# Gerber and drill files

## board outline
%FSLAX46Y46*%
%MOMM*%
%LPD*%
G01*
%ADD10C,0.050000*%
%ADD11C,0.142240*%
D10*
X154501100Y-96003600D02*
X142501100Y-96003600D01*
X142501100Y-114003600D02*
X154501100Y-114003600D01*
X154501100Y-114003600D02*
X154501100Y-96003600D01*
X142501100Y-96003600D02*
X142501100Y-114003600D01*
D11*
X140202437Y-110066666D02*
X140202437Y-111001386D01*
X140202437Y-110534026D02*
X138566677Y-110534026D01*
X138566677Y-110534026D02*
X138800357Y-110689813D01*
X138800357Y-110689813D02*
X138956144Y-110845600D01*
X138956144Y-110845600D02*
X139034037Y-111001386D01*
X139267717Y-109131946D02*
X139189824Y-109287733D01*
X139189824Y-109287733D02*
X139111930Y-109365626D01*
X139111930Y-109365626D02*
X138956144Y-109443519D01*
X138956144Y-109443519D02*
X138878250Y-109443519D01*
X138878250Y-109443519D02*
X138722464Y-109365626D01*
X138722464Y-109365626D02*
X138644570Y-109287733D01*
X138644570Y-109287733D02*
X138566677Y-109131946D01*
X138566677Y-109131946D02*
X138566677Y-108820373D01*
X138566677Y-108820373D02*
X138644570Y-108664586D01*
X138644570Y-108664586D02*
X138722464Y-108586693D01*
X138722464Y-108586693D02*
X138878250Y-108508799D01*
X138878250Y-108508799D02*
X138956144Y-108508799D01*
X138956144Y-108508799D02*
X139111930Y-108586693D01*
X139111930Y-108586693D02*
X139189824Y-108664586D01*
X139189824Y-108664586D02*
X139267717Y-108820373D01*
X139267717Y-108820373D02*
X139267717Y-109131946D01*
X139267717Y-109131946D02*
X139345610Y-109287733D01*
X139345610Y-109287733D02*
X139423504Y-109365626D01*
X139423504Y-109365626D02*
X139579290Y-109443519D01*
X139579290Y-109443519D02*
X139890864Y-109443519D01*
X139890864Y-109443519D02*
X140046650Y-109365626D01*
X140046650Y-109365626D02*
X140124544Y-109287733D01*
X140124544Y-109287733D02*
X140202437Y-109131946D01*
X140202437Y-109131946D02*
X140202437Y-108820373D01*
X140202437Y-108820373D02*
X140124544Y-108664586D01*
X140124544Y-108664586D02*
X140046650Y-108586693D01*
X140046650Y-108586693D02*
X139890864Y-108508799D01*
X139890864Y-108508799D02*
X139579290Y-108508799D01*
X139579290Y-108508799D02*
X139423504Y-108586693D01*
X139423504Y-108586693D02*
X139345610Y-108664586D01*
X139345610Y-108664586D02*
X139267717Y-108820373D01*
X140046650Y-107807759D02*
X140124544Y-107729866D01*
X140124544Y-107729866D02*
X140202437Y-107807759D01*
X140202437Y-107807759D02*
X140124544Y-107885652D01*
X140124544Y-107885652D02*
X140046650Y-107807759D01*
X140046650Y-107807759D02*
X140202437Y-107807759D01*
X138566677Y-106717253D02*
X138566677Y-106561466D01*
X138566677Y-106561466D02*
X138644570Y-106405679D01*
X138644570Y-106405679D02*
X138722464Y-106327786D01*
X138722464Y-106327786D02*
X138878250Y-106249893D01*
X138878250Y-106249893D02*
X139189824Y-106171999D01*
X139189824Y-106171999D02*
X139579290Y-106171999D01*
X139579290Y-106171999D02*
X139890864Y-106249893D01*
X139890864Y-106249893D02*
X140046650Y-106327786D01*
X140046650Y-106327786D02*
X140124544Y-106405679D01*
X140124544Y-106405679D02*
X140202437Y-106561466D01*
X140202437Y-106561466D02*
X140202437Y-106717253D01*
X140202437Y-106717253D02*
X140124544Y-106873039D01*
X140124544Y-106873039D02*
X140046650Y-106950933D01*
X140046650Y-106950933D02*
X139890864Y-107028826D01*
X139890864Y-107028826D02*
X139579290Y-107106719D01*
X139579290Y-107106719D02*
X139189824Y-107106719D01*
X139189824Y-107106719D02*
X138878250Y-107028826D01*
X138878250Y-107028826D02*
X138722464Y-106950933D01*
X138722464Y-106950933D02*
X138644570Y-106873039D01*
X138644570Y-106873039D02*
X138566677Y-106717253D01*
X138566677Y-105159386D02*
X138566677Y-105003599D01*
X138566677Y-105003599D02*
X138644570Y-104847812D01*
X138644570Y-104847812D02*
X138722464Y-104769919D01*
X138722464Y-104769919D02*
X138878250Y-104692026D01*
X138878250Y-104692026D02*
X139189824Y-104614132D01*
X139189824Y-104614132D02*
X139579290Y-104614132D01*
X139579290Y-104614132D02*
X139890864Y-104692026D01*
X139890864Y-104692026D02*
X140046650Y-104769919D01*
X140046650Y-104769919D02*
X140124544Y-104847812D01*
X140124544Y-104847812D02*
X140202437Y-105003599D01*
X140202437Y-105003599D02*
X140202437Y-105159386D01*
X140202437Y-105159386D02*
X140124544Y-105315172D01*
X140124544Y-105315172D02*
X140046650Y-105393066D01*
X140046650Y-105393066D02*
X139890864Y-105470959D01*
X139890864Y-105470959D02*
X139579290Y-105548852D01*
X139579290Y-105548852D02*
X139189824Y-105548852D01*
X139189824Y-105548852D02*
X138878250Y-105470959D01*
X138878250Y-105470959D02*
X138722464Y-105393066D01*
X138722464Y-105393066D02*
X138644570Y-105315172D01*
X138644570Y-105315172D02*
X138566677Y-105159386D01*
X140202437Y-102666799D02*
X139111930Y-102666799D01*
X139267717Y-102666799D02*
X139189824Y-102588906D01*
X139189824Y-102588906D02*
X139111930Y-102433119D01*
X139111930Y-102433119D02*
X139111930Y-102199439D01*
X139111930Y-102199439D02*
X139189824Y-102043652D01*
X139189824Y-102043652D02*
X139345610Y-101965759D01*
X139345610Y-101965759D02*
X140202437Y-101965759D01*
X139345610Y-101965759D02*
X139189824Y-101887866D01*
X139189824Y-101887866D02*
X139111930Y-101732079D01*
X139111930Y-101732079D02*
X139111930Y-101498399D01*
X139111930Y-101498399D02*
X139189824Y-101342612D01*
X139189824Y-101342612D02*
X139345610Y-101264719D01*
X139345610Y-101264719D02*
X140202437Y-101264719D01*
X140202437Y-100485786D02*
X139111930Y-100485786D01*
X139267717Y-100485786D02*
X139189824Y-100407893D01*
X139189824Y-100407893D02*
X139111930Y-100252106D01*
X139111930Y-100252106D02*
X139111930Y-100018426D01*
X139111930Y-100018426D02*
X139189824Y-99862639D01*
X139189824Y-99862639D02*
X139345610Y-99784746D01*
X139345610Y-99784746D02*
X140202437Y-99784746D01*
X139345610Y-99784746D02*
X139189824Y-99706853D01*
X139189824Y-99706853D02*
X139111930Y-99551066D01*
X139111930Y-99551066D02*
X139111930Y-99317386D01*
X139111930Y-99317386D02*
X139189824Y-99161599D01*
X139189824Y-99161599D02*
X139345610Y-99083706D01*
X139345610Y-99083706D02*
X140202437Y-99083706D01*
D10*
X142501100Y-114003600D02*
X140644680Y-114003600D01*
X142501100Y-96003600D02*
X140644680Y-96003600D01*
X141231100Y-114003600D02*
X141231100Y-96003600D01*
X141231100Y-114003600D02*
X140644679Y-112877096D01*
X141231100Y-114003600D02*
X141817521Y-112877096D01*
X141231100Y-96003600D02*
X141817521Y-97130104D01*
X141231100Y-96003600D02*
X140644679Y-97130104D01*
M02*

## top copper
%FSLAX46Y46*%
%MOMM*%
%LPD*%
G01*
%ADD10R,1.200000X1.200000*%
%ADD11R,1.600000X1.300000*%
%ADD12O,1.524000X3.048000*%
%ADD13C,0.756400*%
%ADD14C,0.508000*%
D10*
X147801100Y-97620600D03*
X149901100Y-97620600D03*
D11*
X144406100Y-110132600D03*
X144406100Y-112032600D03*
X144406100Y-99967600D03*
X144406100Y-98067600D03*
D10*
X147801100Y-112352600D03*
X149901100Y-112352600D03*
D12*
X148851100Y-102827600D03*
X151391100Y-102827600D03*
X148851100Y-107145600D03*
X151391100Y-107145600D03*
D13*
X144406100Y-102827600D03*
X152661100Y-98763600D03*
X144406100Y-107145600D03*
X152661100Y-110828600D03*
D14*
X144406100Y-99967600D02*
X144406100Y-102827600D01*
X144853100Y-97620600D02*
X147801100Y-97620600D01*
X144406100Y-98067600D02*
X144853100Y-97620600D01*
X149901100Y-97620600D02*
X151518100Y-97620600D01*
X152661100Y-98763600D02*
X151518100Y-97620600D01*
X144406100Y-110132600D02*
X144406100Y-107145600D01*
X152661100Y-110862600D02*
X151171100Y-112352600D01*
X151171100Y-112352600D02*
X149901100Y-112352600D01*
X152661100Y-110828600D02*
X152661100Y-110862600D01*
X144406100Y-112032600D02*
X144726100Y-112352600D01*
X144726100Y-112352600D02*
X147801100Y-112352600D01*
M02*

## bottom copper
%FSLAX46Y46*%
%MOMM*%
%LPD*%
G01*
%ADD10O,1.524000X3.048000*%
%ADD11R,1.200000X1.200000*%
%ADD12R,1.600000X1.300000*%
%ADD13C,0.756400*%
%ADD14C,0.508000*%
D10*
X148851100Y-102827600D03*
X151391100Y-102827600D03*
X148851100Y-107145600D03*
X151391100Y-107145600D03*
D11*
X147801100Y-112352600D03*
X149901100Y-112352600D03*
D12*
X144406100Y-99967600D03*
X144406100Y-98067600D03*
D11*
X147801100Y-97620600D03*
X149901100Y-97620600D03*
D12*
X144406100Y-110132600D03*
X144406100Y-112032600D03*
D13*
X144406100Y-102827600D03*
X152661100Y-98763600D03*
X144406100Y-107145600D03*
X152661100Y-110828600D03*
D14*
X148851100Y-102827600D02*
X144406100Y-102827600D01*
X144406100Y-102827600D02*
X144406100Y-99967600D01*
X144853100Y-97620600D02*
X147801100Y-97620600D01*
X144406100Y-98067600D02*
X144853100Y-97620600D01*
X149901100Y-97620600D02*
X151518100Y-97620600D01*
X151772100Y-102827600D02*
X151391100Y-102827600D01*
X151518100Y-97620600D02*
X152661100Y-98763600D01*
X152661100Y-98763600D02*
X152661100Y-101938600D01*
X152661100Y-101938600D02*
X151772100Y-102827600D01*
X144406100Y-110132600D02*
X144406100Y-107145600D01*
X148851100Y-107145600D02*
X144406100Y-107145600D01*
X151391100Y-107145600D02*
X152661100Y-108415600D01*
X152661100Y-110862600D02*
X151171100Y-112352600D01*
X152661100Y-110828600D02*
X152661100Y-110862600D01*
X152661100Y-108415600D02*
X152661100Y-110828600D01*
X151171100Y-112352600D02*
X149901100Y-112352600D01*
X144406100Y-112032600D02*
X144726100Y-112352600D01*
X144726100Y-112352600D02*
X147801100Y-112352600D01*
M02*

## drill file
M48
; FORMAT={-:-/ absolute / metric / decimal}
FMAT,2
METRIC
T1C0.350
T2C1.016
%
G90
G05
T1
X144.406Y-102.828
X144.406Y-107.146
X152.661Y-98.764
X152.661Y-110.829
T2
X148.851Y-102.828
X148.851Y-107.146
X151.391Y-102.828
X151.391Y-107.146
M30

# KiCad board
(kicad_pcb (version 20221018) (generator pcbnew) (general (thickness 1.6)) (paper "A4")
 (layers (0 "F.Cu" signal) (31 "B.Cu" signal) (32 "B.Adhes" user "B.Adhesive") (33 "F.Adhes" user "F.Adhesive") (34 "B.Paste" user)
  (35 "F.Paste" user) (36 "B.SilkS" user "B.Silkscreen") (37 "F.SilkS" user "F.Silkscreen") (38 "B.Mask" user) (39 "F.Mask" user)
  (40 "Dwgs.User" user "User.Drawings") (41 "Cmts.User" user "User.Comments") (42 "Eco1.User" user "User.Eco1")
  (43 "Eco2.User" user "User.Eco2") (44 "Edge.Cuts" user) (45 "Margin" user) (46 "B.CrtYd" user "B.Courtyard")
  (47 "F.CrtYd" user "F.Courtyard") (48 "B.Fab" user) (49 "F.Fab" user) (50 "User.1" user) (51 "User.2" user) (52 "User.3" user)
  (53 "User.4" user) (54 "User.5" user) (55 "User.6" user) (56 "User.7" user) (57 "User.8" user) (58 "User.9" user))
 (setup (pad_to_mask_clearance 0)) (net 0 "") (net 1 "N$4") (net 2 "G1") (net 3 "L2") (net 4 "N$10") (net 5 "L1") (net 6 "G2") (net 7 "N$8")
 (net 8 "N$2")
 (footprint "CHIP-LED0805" (layer "F.Cu") (at 148.8511 97.6206 -90)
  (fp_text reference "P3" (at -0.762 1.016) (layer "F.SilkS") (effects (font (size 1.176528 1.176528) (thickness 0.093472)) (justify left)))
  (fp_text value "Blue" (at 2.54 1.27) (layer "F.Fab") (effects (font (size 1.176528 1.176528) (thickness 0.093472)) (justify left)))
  (pad "A" smd rect (at 0 1.05 270) (size 1.2 1.2) (layers "F.Cu" "F.Paste" "F.Mask") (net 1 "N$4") (solder_mask_margin 0.1016)
   (thermal_bridge_angle 45))
  (pad "C" smd rect (at 0 -1.05 270) (size 1.2 1.2) (layers "F.Cu" "F.Paste" "F.Mask") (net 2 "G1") (solder_mask_margin 0.1016)
   (thermal_bridge_angle 45)))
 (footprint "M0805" (layer "F.Cu") (at 144.4061 111.0826 -90)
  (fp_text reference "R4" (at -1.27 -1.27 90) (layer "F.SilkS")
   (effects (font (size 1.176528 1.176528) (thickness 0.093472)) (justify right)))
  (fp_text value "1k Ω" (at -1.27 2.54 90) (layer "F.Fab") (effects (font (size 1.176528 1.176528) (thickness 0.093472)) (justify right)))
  (pad "1" smd rect (at -0.95 0 270) (size 1.3 1.6) (layers "F.Cu" "F.Paste" "F.Mask") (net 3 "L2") (solder_mask_margin 0.1016)
   (thermal_bridge_angle 45))
  (pad "2" smd rect (at 0.95 0 270) (size 1.3 1.6) (layers "F.Cu" "F.Paste" "F.Mask") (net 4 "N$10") (solder_mask_margin 0.1016)
   (thermal_bridge_angle 45)))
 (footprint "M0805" (layer "F.Cu") (at 144.4061 99.0176 90)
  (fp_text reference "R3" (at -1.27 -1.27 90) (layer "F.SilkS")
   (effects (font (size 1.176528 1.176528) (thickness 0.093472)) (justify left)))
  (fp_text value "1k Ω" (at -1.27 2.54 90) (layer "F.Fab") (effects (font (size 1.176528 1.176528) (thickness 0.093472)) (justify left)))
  (pad "1" smd rect (at -0.95 0 90) (size 1.3 1.6) (layers "F.Cu" "F.Paste" "F.Mask") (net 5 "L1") (solder_mask_margin 0.1016)
   (thermal_bridge_angle 45))
  (pad "2" smd rect (at 0.95 0 90) (size 1.3 1.6) (layers "F.Cu" "F.Paste" "F.Mask") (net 1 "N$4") (solder_mask_margin 0.1016)
   (thermal_bridge_angle 45)))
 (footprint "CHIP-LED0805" (layer "F.Cu") (at 148.8511 112.3526 -90)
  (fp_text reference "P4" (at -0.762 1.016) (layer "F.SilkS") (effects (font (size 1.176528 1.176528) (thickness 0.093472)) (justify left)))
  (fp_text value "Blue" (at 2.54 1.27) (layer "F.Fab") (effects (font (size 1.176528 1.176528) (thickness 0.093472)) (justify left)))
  (pad "A" smd rect (at 0 1.05 270) (size 1.2 1.2) (layers "F.Cu" "F.Paste" "F.Mask") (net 4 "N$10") (solder_mask_margin 0.1016)
   (thermal_bridge_angle 45))
  (pad "C" smd rect (at 0 -1.05 270) (size 1.2 1.2) (layers "F.Cu" "F.Paste" "F.Mask") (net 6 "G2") (solder_mask_margin 0.1016)
   (thermal_bridge_angle 45)))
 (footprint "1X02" (layer "F.Cu") (at 150.1211 102.8276)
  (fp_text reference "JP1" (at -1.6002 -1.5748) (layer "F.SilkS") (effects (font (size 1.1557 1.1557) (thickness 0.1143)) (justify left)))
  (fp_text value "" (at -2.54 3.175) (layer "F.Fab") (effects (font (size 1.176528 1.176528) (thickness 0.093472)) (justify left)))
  (pad "1" thru_hole oval (at -1.27 0 90) (size 3.048 1.524) (drill 1.016) (layers "*.Cu" "*.Mask") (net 5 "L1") (solder_mask_margin 0.1016)
   (thermal_bridge_angle 45))
  (pad "2" thru_hole oval (at 1.27 0 90) (size 3.048 1.524) (drill 1.016) (layers "*.Cu" "*.Mask") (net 2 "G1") (solder_mask_margin 0.1016)
   (thermal_bridge_angle 45)))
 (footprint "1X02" (layer "F.Cu") (at 150.1211 107.1456)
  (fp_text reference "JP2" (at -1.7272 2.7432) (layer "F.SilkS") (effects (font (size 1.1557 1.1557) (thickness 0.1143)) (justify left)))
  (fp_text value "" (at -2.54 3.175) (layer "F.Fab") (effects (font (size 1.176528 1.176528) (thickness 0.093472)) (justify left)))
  (pad "1" thru_hole oval (at -1.27 0 90) (size 3.048 1.524) (drill 1.016) (layers "*.Cu" "*.Mask") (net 3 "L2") (solder_mask_margin 0.1016)
   (thermal_bridge_angle 45))
  (pad "2" thru_hole oval (at 1.27 0 90) (size 3.048 1.524) (drill 1.016) (layers "*.Cu" "*.Mask") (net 6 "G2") (solder_mask_margin 0.1016)
   (thermal_bridge_angle 45)))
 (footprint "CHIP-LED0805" (layer "B.Cu") (at 148.8511 112.3526 90)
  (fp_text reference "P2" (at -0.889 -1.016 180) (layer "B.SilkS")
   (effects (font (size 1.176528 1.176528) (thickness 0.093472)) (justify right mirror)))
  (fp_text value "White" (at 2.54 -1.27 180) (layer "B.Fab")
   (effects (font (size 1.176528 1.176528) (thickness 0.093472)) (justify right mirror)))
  (pad "A" smd rect (at 0 -1.05 90) (size 1.2 1.2) (layers "B.Cu" "B.Paste" "B.Mask") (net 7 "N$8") (solder_mask_margin 0.1016)
   (thermal_bridge_angle 45))
  (pad "C" smd rect (at 0 1.05 90) (size 1.2 1.2) (layers "B.Cu" "B.Paste" "B.Mask") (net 6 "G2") (solder_mask_margin 0.1016)
   (thermal_bridge_angle 45)))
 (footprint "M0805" (layer "B.Cu") (at 144.4061 99.0176 90)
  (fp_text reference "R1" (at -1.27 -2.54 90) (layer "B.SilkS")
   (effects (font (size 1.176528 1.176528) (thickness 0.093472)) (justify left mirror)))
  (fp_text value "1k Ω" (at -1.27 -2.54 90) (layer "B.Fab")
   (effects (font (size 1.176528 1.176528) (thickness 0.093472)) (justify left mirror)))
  (pad "1" smd rect (at -0.95 0 90) (size 1.3 1.6) (layers "B.Cu" "B.Paste" "B.Mask") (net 5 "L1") (solder_mask_margin 0.1016)
   (thermal_bridge_angle 45))
  (pad "2" smd rect (at 0.95 0 90) (size 1.3 1.6) (layers "B.Cu" "B.Paste" "B.Mask") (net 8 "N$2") (solder_mask_margin 0.1016)
   (thermal_bridge_angle 45)))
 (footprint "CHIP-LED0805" (layer "B.Cu") (at 148.8511 97.6206 90)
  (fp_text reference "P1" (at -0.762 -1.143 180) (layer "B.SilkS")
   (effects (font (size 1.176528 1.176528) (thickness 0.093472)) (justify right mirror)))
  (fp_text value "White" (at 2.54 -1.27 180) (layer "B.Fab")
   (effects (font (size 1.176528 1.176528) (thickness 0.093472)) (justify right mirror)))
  (pad "A" smd rect (at 0 -1.05 90) (size 1.2 1.2) (layers "B.Cu" "B.Paste" "B.Mask") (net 8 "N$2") (solder_mask_margin 0.1016)
   (thermal_bridge_angle 45))
  (pad "C" smd rect (at 0 1.05 90) (size 1.2 1.2) (layers "B.Cu" "B.Paste" "B.Mask") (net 2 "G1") (solder_mask_margin 0.1016)
   (thermal_bridge_angle 45)))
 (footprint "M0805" (layer "B.Cu") (at 144.4061 111.0826 -90)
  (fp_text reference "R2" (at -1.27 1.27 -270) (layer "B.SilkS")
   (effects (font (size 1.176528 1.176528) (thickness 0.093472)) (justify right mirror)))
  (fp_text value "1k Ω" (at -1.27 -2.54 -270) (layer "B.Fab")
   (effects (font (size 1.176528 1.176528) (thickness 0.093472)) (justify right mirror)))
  (pad "1" smd rect (at -0.95 0 270) (size 1.3 1.6) (layers "B.Cu" "B.Paste" "B.Mask") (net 3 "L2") (solder_mask_margin 0.1016)
   (thermal_bridge_angle 45))
  (pad "2" smd rect (at 0.95 0 270) (size 1.3 1.6) (layers "B.Cu" "B.Paste" "B.Mask") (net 7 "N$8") (solder_mask_margin 0.1016)
   (thermal_bridge_angle 45)))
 (gr_line (start 154.5011 96.0036) (end 142.5011 96.0036) (stroke (width 0.05) (type solid)) (layer "Edge.Cuts"))
 (gr_line (start 142.5011 114.0036) (end 154.5011 114.0036) (stroke (width 0.05) (type solid)) (layer "Edge.Cuts"))
 (gr_line (start 154.5011 114.0036) (end 154.5011 96.0036) (stroke (width 0.05) (type solid)) (layer "Edge.Cuts"))
 (gr_line (start 142.5011 96.0036) (end 142.5011 114.0036) (stroke (width 0.05) (type solid)) (layer "Edge.Cuts"))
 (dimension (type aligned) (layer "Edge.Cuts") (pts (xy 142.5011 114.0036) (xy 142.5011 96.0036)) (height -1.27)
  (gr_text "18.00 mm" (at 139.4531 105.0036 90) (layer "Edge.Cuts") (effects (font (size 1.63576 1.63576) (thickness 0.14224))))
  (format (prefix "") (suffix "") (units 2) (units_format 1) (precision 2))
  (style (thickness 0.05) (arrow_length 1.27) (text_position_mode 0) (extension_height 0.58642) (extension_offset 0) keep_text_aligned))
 (segment (start 144.4061 99.9676) (end 144.4061 102.8276) (width 0.508) (layer "F.Cu") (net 5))
 (via (at 144.4061 102.8276) (size 0.7564) (drill 0.35) (layers "F.Cu" "B.Cu") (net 5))
 (segment (start 148.8511 102.8276) (end 144.4061 102.8276) (width 0.508) (layer "B.Cu") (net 5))
 (segment (start 144.4061 102.8276) (end 144.4061 99.9676) (width 0.508) (layer "B.Cu") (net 5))
 (segment (start 144.8531 97.6206) (end 147.8011 97.6206) (width 0.508) (layer "B.Cu") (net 8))
 (segment (start 144.4061 98.0676) (end 144.8531 97.6206) (width 0.508) (layer "B.Cu") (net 8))
 (segment (start 144.8531 97.6206) (end 147.8011 97.6206) (width 0.508) (layer "F.Cu") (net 1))
 (segment (start 144.4061 98.0676) (end 144.8531 97.6206) (width 0.508) (layer "F.Cu") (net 1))
 (segment (start 149.9011 97.6206) (end 151.5181 97.6206) (width 0.508) (layer "F.Cu") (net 2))
 (segment (start 152.6611 98.7636) (end 151.5181 97.6206) (width 0.508) (layer "F.Cu") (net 2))
 (via (at 152.6611 98.7636) (size 0.7564) (drill 0.35) (layers "F.Cu" "B.Cu") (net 2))
 (segment (start 149.9011 97.6206) (end 151.5181 97.6206) (width 0.508) (layer "B.Cu") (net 2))
 (segment (start 151.7721 102.8276) (end 151.3911 102.8276) (width 0.508) (layer "B.Cu") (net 2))
 (segment (start 151.5181 97.6206) (end 152.6611 98.7636) (width 0.508) (layer "B.Cu") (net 2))
 (segment (start 152.6611 98.7636) (end 152.6611 101.9386) (width 0.508) (layer "B.Cu") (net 2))
 (segment (start 152.6611 101.9386) (end 151.7721 102.8276) (width 0.508) (layer "B.Cu") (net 2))
 (segment (start 144.4061 110.1326) (end 144.4061 107.1456) (width 0.508) (layer "F.Cu") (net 3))
 (via (at 144.4061 107.1456) (size 0.7564) (drill 0.35) (layers "F.Cu" "B.Cu") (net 3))
 (segment (start 144.4061 110.1326) (end 144.4061 107.1456) (width 0.508) (layer "B.Cu") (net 3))
 (segment (start 148.8511 107.1456) (end 144.4061 107.1456) (width 0.508) (layer "B.Cu") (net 3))
 (segment (start 152.6611 110.8626) (end 151.1711 112.3526) (width 0.508) (layer "F.Cu") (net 6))
 (segment (start 151.1711 112.3526) (end 149.9011 112.3526) (width 0.508) (layer "F.Cu") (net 6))
 (segment (start 152.6611 110.8286) (end 152.6611 110.8626) (width 0.508) (layer "F.Cu") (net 6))
 (via (at 152.6611 110.8286) (size 0.7564) (drill 0.35) (layers "F.Cu" "B.Cu") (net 6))
 (segment (start 151.3911 107.1456) (end 152.6611 108.4156) (width 0.508) (layer "B.Cu") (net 6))
 (segment (start 152.6611 110.8626) (end 151.1711 112.3526) (width 0.508) (layer "B.Cu") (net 6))
 (segment (start 152.6611 110.8286) (end 152.6611 110.8626) (width 0.508) (layer "B.Cu") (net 6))
 (segment (start 152.6611 108.4156) (end 152.6611 110.8286) (width 0.508) (layer "B.Cu") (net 6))
 (segment (start 151.1711 112.3526) (end 149.9011 112.3526) (width 0.508) (layer "B.Cu") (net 6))
 (segment (start 144.4061 112.0326) (end 144.7261 112.3526) (width 0.508) (layer "B.Cu") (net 7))
 (segment (start 144.7261 112.3526) (end 147.8011 112.3526) (width 0.508) (layer "B.Cu") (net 7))
 (segment (start 144.4061 112.0326) (end 144.7261 112.3526) (width 0.508) (layer "F.Cu") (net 4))
 (segment (start 144.7261 112.3526) (end 147.8011 112.3526) (width 0.508) (layer "F.Cu") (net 4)))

